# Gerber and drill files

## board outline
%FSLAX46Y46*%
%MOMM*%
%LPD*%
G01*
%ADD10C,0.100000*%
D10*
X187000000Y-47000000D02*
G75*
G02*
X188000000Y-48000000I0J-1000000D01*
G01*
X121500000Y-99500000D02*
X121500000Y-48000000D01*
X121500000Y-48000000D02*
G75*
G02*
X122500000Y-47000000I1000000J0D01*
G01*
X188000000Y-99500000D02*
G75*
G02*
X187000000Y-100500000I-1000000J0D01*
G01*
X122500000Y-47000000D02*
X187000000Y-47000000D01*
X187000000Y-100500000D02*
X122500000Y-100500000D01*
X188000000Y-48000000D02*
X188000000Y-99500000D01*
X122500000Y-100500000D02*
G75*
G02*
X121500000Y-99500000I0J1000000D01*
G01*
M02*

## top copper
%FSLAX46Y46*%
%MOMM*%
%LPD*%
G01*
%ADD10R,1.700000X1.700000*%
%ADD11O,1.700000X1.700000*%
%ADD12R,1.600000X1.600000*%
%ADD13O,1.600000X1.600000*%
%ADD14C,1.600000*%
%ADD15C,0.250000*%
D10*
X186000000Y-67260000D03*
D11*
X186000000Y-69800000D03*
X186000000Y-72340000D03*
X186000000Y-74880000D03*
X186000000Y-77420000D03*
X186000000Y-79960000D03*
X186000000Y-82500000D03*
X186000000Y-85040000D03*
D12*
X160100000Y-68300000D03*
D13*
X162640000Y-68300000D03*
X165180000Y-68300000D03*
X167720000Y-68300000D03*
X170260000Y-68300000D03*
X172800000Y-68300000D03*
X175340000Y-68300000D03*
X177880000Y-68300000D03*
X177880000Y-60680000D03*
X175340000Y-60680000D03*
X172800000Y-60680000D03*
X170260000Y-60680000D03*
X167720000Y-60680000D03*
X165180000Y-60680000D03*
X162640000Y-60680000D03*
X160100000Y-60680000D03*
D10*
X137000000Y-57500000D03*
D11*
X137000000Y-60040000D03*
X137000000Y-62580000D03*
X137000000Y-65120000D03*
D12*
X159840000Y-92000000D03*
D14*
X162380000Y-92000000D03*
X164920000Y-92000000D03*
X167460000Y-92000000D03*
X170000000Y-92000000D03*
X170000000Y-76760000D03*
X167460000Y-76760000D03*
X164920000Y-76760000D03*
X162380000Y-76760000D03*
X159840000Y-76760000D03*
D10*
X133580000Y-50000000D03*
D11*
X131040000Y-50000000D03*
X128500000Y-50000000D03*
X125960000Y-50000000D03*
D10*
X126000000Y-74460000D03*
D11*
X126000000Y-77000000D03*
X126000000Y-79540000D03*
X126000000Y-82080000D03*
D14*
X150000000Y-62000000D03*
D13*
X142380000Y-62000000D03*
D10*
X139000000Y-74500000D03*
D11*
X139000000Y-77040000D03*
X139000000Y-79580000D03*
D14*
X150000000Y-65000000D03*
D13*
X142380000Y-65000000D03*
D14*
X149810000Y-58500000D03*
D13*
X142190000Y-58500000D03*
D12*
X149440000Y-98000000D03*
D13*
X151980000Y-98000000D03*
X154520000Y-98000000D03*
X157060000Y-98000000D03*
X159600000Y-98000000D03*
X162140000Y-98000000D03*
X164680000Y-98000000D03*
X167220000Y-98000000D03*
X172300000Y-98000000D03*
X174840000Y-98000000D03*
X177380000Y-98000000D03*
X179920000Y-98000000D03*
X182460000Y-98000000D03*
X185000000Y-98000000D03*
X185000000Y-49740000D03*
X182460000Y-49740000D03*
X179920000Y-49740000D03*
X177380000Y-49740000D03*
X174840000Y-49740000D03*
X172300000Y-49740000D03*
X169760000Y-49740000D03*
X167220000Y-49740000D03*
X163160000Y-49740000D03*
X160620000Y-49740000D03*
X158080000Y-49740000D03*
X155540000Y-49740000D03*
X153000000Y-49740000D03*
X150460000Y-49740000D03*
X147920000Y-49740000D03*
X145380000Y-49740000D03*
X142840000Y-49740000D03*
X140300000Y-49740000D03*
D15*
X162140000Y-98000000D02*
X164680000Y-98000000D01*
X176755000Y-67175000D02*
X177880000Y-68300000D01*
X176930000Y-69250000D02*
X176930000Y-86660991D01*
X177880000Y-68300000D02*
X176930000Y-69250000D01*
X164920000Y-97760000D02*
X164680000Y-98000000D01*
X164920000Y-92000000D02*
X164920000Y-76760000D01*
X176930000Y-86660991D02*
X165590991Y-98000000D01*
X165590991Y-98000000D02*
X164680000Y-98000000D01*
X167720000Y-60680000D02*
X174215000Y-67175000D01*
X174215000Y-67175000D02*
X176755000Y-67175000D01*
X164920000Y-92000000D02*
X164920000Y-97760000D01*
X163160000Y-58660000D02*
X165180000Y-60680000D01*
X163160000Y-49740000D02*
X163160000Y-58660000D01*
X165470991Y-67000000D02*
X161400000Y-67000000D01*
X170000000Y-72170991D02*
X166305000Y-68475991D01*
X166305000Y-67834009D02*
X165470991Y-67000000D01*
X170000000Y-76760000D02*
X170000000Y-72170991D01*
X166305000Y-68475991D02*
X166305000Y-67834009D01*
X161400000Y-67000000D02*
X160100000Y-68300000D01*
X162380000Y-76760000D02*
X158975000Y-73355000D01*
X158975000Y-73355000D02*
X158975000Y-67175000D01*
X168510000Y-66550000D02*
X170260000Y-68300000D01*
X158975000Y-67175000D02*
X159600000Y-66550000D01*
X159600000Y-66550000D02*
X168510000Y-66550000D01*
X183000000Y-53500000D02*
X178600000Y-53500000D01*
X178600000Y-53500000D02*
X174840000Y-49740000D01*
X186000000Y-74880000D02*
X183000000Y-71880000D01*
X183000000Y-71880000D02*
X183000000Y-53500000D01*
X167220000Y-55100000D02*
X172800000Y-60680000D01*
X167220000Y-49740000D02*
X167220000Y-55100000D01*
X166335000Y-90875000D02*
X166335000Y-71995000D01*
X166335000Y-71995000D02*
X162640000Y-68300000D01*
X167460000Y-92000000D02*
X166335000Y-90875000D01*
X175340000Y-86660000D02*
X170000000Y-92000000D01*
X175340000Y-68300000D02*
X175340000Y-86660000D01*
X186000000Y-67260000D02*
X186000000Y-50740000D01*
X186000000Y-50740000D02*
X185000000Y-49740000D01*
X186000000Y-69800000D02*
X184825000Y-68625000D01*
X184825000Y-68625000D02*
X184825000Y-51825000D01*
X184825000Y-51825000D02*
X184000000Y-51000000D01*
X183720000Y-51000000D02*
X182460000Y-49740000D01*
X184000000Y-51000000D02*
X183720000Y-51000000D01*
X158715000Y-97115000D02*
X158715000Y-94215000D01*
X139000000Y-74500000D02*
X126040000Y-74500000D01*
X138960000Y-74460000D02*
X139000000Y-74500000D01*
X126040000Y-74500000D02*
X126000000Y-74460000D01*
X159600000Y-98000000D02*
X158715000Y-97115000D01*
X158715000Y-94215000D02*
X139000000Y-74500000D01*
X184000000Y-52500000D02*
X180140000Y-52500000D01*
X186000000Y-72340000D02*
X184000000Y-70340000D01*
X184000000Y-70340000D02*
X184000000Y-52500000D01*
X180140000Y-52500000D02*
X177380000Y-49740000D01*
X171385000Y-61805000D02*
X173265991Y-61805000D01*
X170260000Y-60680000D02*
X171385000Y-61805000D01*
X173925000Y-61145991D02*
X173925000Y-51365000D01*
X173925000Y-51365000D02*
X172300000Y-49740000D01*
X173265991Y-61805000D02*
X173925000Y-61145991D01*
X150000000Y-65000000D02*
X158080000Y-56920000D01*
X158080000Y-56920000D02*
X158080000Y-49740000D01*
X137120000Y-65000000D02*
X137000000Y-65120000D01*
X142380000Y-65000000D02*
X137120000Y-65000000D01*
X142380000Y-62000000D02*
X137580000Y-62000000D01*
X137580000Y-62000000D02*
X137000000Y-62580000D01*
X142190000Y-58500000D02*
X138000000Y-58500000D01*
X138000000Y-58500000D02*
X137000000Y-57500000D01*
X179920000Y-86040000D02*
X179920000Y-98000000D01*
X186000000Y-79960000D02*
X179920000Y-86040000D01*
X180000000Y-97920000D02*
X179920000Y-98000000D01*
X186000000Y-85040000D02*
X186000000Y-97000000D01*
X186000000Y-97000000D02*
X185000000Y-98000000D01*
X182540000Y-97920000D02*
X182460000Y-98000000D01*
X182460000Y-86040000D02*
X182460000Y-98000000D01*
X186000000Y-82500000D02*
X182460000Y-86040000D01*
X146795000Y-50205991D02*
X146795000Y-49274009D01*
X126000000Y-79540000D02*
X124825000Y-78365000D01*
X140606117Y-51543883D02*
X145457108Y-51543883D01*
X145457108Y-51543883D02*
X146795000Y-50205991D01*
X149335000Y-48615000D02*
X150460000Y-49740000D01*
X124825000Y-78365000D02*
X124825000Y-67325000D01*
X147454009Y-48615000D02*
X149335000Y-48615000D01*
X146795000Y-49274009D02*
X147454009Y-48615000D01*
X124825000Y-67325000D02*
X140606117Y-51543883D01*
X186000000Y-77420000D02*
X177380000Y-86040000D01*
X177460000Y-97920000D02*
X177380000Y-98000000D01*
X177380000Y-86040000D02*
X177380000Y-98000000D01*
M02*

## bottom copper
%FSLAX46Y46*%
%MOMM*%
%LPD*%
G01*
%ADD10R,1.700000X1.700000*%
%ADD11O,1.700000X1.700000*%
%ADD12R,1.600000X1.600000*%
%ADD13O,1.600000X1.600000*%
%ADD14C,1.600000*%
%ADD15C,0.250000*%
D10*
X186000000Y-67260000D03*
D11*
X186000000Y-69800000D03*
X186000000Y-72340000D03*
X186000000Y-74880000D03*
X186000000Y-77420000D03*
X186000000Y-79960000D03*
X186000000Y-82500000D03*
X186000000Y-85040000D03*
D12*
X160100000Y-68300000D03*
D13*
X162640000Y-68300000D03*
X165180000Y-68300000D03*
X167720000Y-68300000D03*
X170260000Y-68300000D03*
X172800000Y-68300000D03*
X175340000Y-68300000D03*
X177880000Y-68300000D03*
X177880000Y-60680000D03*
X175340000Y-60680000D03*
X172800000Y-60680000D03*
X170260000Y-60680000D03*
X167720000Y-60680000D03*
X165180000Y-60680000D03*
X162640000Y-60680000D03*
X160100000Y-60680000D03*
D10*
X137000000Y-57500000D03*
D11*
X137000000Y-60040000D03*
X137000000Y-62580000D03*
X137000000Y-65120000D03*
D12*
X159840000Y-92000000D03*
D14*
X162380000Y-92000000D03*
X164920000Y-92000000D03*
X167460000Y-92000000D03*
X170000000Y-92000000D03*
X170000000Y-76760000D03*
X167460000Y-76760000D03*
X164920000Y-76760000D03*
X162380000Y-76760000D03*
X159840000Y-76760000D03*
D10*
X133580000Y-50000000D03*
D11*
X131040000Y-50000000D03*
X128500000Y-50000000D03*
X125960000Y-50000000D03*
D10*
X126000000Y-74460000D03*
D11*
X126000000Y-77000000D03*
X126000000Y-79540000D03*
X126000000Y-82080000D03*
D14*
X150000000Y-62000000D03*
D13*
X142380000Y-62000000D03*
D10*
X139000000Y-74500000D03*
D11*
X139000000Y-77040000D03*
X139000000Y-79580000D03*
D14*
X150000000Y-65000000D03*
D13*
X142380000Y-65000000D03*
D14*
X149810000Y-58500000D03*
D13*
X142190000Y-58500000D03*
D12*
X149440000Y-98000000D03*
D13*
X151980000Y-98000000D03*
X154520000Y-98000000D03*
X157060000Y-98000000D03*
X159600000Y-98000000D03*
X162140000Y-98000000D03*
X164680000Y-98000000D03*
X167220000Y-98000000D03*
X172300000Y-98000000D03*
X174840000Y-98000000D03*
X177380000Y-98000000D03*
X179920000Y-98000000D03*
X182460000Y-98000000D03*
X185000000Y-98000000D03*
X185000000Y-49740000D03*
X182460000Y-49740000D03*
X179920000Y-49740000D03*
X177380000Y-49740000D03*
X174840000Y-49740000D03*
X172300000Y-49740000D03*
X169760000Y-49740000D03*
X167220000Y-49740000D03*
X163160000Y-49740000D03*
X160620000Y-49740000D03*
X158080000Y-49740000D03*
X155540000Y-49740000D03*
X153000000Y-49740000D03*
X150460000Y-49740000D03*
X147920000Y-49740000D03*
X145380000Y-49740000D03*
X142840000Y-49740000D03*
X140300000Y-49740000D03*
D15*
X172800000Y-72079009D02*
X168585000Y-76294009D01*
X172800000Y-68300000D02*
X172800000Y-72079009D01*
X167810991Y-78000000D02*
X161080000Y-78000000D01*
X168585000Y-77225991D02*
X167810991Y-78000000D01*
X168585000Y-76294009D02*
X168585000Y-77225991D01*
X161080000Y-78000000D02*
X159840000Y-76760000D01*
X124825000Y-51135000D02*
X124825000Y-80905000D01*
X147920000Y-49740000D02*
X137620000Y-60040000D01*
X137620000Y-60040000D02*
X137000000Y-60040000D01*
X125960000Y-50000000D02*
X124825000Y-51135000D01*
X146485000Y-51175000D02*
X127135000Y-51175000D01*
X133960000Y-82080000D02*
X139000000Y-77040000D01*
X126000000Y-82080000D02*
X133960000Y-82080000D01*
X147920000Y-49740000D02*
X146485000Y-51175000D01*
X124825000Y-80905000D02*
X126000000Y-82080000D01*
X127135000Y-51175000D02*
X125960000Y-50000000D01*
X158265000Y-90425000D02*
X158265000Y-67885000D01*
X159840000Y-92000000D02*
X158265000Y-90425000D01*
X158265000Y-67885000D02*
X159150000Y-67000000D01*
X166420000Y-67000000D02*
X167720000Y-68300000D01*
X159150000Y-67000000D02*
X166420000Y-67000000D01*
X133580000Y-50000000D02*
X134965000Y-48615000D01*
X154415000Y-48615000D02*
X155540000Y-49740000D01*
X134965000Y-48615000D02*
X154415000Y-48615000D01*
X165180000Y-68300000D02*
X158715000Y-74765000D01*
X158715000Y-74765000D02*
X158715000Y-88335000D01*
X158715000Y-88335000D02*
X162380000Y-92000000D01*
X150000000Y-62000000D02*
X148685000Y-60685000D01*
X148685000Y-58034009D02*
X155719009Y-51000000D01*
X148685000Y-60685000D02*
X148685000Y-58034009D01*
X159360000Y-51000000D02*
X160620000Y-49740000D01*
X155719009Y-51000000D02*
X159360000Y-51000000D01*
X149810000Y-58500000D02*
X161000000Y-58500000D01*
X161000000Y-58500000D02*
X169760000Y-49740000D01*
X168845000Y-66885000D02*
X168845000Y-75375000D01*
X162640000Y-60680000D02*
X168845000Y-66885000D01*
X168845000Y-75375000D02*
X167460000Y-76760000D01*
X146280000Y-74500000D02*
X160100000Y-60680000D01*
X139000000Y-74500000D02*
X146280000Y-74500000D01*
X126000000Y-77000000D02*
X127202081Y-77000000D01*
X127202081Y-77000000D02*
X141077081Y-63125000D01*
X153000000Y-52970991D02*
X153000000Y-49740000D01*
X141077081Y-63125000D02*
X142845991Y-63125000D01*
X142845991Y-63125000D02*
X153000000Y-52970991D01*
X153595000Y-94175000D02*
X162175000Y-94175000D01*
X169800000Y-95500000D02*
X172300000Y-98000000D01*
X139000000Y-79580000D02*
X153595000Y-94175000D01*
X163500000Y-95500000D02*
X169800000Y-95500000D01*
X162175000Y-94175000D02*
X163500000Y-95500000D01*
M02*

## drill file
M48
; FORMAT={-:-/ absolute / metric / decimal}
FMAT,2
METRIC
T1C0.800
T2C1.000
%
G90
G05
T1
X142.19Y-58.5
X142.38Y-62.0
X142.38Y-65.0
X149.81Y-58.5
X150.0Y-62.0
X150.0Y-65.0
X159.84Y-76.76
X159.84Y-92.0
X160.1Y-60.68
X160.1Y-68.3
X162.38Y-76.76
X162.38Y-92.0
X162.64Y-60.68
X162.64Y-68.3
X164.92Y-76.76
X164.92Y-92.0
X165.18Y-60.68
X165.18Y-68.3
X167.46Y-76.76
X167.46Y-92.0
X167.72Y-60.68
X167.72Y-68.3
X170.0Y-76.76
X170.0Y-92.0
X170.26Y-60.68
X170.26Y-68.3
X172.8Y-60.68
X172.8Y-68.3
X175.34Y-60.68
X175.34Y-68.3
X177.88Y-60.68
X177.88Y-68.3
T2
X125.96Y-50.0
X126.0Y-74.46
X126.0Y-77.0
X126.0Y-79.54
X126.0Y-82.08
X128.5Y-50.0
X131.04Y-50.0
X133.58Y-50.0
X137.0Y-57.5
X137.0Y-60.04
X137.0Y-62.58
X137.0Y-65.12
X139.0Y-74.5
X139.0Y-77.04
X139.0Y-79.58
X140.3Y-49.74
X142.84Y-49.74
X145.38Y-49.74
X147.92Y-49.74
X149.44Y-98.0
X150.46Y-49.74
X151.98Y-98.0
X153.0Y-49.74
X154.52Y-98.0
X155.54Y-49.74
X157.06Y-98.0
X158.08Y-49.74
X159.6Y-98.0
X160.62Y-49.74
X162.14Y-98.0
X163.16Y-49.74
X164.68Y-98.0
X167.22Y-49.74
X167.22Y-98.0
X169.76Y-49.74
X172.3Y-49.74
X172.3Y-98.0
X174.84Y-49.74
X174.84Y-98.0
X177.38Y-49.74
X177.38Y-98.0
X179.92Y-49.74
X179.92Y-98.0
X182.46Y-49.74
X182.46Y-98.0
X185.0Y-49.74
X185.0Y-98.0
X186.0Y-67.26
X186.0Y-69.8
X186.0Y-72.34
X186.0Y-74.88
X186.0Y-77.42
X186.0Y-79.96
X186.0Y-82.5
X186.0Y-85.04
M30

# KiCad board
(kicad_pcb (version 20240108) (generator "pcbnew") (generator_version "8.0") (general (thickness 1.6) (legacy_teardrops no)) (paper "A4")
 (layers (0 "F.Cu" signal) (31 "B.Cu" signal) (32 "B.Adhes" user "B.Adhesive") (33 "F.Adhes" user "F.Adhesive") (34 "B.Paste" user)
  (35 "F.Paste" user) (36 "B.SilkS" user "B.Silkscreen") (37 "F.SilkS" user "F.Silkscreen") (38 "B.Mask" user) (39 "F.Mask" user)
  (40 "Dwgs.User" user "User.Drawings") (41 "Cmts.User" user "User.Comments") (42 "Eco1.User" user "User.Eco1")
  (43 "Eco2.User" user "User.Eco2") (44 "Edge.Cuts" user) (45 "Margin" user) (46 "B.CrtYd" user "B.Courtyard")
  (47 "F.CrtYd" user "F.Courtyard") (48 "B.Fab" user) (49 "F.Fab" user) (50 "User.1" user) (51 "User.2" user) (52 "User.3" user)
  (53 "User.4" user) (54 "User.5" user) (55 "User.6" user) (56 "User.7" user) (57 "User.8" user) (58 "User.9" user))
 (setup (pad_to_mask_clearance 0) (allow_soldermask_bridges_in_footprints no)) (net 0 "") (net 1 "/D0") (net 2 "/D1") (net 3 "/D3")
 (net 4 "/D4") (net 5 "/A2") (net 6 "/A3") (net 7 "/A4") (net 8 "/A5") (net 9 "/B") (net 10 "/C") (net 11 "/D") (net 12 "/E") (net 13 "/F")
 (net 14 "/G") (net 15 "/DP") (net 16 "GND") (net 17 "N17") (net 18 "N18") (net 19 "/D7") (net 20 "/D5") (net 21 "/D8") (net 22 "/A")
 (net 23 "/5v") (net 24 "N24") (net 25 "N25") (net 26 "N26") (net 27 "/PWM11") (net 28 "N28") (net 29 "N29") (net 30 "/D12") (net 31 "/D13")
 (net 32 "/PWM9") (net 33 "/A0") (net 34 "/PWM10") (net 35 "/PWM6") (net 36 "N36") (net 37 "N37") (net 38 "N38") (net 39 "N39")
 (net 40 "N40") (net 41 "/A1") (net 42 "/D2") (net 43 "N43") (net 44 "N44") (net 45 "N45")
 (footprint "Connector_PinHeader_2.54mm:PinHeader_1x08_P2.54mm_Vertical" (layer "F.Cu") (at 186 67.26)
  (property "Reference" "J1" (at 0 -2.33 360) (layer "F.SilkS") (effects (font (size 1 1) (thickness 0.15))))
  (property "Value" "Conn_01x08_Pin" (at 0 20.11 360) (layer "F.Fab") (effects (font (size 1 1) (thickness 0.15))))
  (pad "1" thru_hole rect (at 0 0) (size 1.7 1.7) (drill 1) (layers "*.Cu" "*.Mask") (remove_unused_layers no) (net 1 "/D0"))
  (pad "2" thru_hole oval (at 0 2.54) (size 1.7 1.7) (drill 1) (layers "*.Cu" "*.Mask") (remove_unused_layers no) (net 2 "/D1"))
  (pad "3" thru_hole oval (at 0 5.08) (size 1.7 1.7) (drill 1) (layers "*.Cu" "*.Mask") (remove_unused_layers no) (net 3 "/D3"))
  (pad "4" thru_hole oval (at 0 7.62) (size 1.7 1.7) (drill 1) (layers "*.Cu" "*.Mask") (remove_unused_layers no) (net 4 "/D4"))
  (pad "5" thru_hole oval (at 0 10.16) (size 1.7 1.7) (drill 1) (layers "*.Cu" "*.Mask") (remove_unused_layers no) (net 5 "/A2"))
  (pad "6" thru_hole oval (at 0 12.7) (size 1.7 1.7) (drill 1) (layers "*.Cu" "*.Mask") (remove_unused_layers no) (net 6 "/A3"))
  (pad "7" thru_hole oval (at 0 15.24) (size 1.7 1.7) (drill 1) (layers "*.Cu" "*.Mask") (remove_unused_layers no) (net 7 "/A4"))
  (pad "8" thru_hole oval (at 0 17.78) (size 1.7 1.7) (drill 1) (layers "*.Cu" "*.Mask") (remove_unused_layers no) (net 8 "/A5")))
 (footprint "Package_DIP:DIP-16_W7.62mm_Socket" (layer "F.Cu") (at 160.1 68.3 90)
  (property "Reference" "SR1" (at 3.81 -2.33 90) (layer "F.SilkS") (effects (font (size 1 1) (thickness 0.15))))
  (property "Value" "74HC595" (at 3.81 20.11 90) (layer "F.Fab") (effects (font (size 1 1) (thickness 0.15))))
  (pad "1" thru_hole rect (at 0 0 90) (size 1.6 1.6) (drill 0.8) (layers "*.Cu" "*.Mask") (remove_unused_layers no) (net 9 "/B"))
  (pad "2" thru_hole oval (at 0 2.54 90) (size 1.6 1.6) (drill 0.8) (layers "*.Cu" "*.Mask") (remove_unused_layers no) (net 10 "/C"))
  (pad "3" thru_hole oval (at 0 5.08 90) (size 1.6 1.6) (drill 0.8) (layers "*.Cu" "*.Mask") (remove_unused_layers no) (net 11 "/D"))
  (pad "4" thru_hole oval (at 0 7.62 90) (size 1.6 1.6) (drill 0.8) (layers "*.Cu" "*.Mask") (remove_unused_layers no) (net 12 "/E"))
  (pad "5" thru_hole oval (at 0 10.16 90) (size 1.6 1.6) (drill 0.8) (layers "*.Cu" "*.Mask") (remove_unused_layers no) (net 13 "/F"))
  (pad "6" thru_hole oval (at 0 12.7 90) (size 1.6 1.6) (drill 0.8) (layers "*.Cu" "*.Mask") (remove_unused_layers no) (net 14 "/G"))
  (pad "7" thru_hole oval (at 0 15.24 90) (size 1.6 1.6) (drill 0.8) (layers "*.Cu" "*.Mask") (remove_unused_layers no) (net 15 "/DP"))
  (pad "8" thru_hole oval (at 0 17.78 90) (size 1.6 1.6) (drill 0.8) (layers "*.Cu" "*.Mask") (remove_unused_layers no) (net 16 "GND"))
  (pad "9" thru_hole oval (at 7.62 17.78 90) (size 1.6 1.6) (drill 0.8) (layers "*.Cu" "*.Mask") (remove_unused_layers no) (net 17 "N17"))
  (pad "10" thru_hole oval (at 7.62 15.24 90) (size 1.6 1.6) (drill 0.8) (layers "*.Cu" "*.Mask") (remove_unused_layers no) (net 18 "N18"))
  (pad "11" thru_hole oval (at 7.62 12.7 90) (size 1.6 1.6) (drill 0.8) (layers "*.Cu" "*.Mask") (remove_unused_layers no) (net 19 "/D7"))
  (pad "12" thru_hole oval (at 7.62 10.16 90) (size 1.6 1.6) (drill 0.8) (layers "*.Cu" "*.Mask") (remove_unused_layers no) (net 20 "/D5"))
  (pad "13" thru_hole oval (at 7.62 7.62 90) (size 1.6 1.6) (drill 0.8) (layers "*.Cu" "*.Mask") (remove_unused_layers no) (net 16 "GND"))
  (pad "14" thru_hole oval (at 7.62 5.08 90) (size 1.6 1.6) (drill 0.8) (layers "*.Cu" "*.Mask") (remove_unused_layers no) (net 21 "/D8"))
  (pad "15" thru_hole oval (at 7.62 2.54 90) (size 1.6 1.6) (drill 0.8) (layers "*.Cu" "*.Mask") (remove_unused_layers no) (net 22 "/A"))
  (pad "16" thru_hole oval (at 7.62 0 90) (size 1.6 1.6) (drill 0.8) (layers "*.Cu" "*.Mask") (remove_unused_layers no) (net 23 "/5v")))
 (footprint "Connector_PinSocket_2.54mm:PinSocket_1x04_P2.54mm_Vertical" (layer "F.Cu") (at 137 57.5)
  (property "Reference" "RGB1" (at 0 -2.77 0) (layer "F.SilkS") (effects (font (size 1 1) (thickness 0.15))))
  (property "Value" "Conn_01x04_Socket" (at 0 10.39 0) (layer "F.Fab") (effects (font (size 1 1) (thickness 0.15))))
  (pad "1" thru_hole rect (at 0 0) (size 1.7 1.7) (drill 1) (layers "*.Cu" "*.Mask") (remove_unused_layers no) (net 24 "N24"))
  (pad "2" thru_hole oval (at 0 2.54) (size 1.7 1.7) (drill 1) (layers "*.Cu" "*.Mask") (remove_unused_layers no) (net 16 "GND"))
  (pad "3" thru_hole oval (at 0 5.08) (size 1.7 1.7) (drill 1) (layers "*.Cu" "*.Mask") (remove_unused_layers no) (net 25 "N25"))
  (pad "4" thru_hole oval (at 0 7.62) (size 1.7 1.7) (drill 1) (layers "*.Cu" "*.Mask") (remove_unused_layers no) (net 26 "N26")))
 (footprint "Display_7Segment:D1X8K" (layer "F.Cu") (at 159.84 92 90)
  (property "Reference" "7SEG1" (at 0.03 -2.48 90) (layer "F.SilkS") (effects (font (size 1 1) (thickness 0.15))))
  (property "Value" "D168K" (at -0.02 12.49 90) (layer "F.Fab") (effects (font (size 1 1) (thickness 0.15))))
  (pad "1" thru_hole rect (at 0 0) (size 1.6 1.6) (drill 0.8) (layers "*.Cu" "*.Mask") (remove_unused_layers no) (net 12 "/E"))
  (pad "2" thru_hole circle (at 0 2.54) (size 1.6 1.6) (drill 0.8) (layers "*.Cu" "*.Mask") (remove_unused_layers no) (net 11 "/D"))
  (pad "3" thru_hole circle (at 0 5.08) (size 1.6 1.6) (drill 0.8) (layers "*.Cu" "*.Mask") (remove_unused_layers no) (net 16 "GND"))
  (pad "4" thru_hole circle (at 0 7.62) (size 1.6 1.6) (drill 0.8) (layers "*.Cu" "*.Mask") (remove_unused_layers no) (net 10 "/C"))
  (pad "5" thru_hole circle (at 0 10.16) (size 1.6 1.6) (drill 0.8) (layers "*.Cu" "*.Mask") (remove_unused_layers no) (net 15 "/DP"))
  (pad "6" thru_hole circle (at 15.24 10.16) (size 1.6 1.6) (drill 0.8) (layers "*.Cu" "*.Mask") (remove_unused_layers no) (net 9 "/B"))
  (pad "7" thru_hole circle (at 15.24 7.62) (size 1.6 1.6) (drill 0.8) (layers "*.Cu" "*.Mask") (remove_unused_layers no) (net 22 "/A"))
  (pad "8" thru_hole circle (at 15.24 5.08) (size 1.6 1.6) (drill 0.8) (layers "*.Cu" "*.Mask") (remove_unused_layers no) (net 16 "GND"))
  (pad "9" thru_hole circle (at 15.24 2.54) (size 1.6 1.6) (drill 0.8) (layers "*.Cu" "*.Mask") (remove_unused_layers no) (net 13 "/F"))
  (pad "10" thru_hole circle (at 15.24 0) (size 1.6 1.6) (drill 0.8) (layers "*.Cu" "*.Mask") (remove_unused_layers no) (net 14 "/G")))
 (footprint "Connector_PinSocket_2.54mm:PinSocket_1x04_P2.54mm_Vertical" (layer "F.Cu") (at 133.58 50 -90)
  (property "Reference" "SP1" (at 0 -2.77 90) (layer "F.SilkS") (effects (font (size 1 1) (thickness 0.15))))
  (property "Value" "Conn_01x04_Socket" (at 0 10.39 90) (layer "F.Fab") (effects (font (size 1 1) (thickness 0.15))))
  (pad "1" thru_hole rect (at 0 0 270) (size 1.7 1.7) (drill 1) (layers "*.Cu" "*.Mask") (remove_unused_layers no) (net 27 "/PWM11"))
  (pad "2" thru_hole oval (at 0 2.54 270) (size 1.7 1.7) (drill 1) (layers "*.Cu" "*.Mask") (remove_unused_layers no) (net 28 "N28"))
  (pad "3" thru_hole oval (at 0 5.08 270) (size 1.7 1.7) (drill 1) (layers "*.Cu" "*.Mask") (remove_unused_layers no) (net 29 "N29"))
  (pad "4" thru_hole oval (at 0 7.62 270) (size 1.7 1.7) (drill 1) (layers "*.Cu" "*.Mask") (remove_unused_layers no) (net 16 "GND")))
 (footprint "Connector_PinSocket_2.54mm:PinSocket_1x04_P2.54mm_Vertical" (layer "F.Cu") (at 126 74.46)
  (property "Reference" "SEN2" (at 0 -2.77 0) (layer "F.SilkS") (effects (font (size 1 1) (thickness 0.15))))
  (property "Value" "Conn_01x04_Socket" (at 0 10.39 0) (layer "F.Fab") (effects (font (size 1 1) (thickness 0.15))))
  (pad "1" thru_hole rect (at 0 0) (size 1.7 1.7) (drill 1) (layers "*.Cu" "*.Mask") (remove_unused_layers no) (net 23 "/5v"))
  (pad "2" thru_hole oval (at 0 2.54) (size 1.7 1.7) (drill 1) (layers "*.Cu" "*.Mask") (remove_unused_layers no) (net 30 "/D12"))
  (pad "3" thru_hole oval (at 0 5.08) (size 1.7 1.7) (drill 1) (layers "*.Cu" "*.Mask") (remove_unused_layers no) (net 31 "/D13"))
  (pad "4" thru_hole oval (at 0 7.62) (size 1.7 1.7) (drill 1) (layers "*.Cu" "*.Mask") (remove_unused_layers no) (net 16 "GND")))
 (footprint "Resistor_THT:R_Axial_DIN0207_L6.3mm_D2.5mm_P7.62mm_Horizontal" (layer "F.Cu") (at 150 62 180)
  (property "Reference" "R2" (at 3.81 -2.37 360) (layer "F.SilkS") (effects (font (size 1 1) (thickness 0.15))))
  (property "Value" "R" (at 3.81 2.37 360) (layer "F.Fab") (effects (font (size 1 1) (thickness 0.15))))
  (pad "1" thru_hole circle (at 0 0 180) (size 1.6 1.6) (drill 0.8) (layers "*.Cu" "*.Mask") (remove_unused_layers no) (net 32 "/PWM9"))
  (pad "2" thru_hole oval (at 7.62 0 180) (size 1.6 1.6) (drill 0.8) (layers "*.Cu" "*.Mask") (remove_unused_layers no) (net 25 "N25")))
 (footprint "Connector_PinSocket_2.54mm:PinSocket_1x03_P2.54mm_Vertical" (layer "F.Cu") (at 139 74.5)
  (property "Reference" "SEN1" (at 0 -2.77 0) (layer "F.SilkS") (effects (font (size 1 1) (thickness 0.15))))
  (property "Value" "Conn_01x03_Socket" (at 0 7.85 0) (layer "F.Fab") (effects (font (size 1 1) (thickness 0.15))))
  (pad "1" thru_hole rect (at 0 0) (size 1.7 1.7) (drill 1) (layers "*.Cu" "*.Mask") (remove_unused_layers no) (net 23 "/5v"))
  (pad "2" thru_hole oval (at 0 2.54) (size 1.7 1.7) (drill 1) (layers "*.Cu" "*.Mask") (remove_unused_layers no) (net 16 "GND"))
  (pad "3" thru_hole oval (at 0 5.08) (size 1.7 1.7) (drill 1) (layers "*.Cu" "*.Mask") (remove_unused_layers no) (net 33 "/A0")))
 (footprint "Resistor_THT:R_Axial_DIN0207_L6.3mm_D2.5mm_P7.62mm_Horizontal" (layer "F.Cu") (at 150 65 180)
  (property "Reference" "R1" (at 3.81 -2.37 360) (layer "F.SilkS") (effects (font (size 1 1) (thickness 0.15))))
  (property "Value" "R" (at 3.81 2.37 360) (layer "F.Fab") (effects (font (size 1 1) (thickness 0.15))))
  (pad "1" thru_hole circle (at 0 0 180) (size 1.6 1.6) (drill 0.8) (layers "*.Cu" "*.Mask") (remove_unused_layers no) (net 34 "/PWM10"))
  (pad "2" thru_hole oval (at 7.62 0 180) (size 1.6 1.6) (drill 0.8) (layers "*.Cu" "*.Mask") (remove_unused_layers no) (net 26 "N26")))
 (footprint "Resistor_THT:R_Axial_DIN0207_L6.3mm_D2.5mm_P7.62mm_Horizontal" (layer "F.Cu") (at 149.81 58.5 180)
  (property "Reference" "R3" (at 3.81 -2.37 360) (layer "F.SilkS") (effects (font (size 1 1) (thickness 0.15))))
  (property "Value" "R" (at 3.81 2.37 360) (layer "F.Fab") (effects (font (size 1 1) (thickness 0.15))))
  (pad "1" thru_hole circle (at 0 0 180) (size 1.6 1.6) (drill 0.8) (layers "*.Cu" "*.Mask") (remove_unused_layers no) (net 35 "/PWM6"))
  (pad "2" thru_hole oval (at 7.62 0 180) (size 1.6 1.6) (drill 0.8) (layers "*.Cu" "*.Mask") (remove_unused_layers no) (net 24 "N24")))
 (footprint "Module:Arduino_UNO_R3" (layer "B.Cu") (at 149.44 98)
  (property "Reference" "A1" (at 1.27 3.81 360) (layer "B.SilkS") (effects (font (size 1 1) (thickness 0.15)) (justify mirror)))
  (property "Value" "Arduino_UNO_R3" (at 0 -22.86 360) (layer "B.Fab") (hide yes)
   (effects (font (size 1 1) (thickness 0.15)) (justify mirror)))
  (pad "1" thru_hole rect (at 0 0 270) (size 1.6 1.6) (drill 1) (layers "*.Cu" "*.Mask") (remove_unused_layers no) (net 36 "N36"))
  (pad "2" thru_hole oval (at 2.54 0 270) (size 1.6 1.6) (drill 1) (layers "*.Cu" "*.Mask") (remove_unused_layers no) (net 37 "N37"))
  (pad "3" thru_hole oval (at 5.08 0 270) (size 1.6 1.6) (drill 1) (layers "*.Cu" "*.Mask") (remove_unused_layers no) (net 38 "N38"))
  (pad "4" thru_hole oval (at 7.62 0 270) (size 1.6 1.6) (drill 1) (layers "*.Cu" "*.Mask") (remove_unused_layers no) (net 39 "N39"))
  (pad "5" thru_hole oval (at 10.16 0 270) (size 1.6 1.6) (drill 1) (layers "*.Cu" "*.Mask") (remove_unused_layers no) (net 23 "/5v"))
  (pad "6" thru_hole oval (at 12.7 0 270) (size 1.6 1.6) (drill 1) (layers "*.Cu" "*.Mask") (remove_unused_layers no) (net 16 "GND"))
  (pad "7" thru_hole oval (at 15.24 0 270) (size 1.6 1.6) (drill 1) (layers "*.Cu" "*.Mask") (remove_unused_layers no) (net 16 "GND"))
  (pad "8" thru_hole oval (at 17.78 0 270) (size 1.6 1.6) (drill 1) (layers "*.Cu" "*.Mask") (remove_unused_layers no) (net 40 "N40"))
  (pad "9" thru_hole oval (at 22.86 0 270) (size 1.6 1.6) (drill 1) (layers "*.Cu" "*.Mask") (remove_unused_layers no) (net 33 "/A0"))
  (pad "10" thru_hole oval (at 25.4 0 270) (size 1.6 1.6) (drill 1) (layers "*.Cu" "*.Mask") (remove_unused_layers no) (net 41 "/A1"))
  (pad "11" thru_hole oval (at 27.94 0 270) (size 1.6 1.6) (drill 1) (layers "*.Cu" "*.Mask") (remove_unused_layers no) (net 5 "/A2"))
  (pad "12" thru_hole oval (at 30.48 0 270) (size 1.6 1.6) (drill 1) (layers "*.Cu" "*.Mask") (remove_unused_layers no) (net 6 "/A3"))
  (pad "13" thru_hole oval (at 33.02 0 270) (size 1.6 1.6) (drill 1) (layers "*.Cu" "*.Mask") (remove_unused_layers no) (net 7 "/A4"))
  (pad "14" thru_hole oval (at 35.56 0 270) (size 1.6 1.6) (drill 1) (layers "*.Cu" "*.Mask") (remove_unused_layers no) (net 8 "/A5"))
  (pad "15" thru_hole oval (at 35.56 -48.26 270) (size 1.6 1.6) (drill 1) (layers "*.Cu" "*.Mask") (remove_unused_layers no) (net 1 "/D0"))
  (pad "16" thru_hole oval (at 33.02 -48.26 270) (size 1.6 1.6) (drill 1) (layers "*.Cu" "*.Mask") (remove_unused_layers no) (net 2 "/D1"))
  (pad "17" thru_hole oval (at 30.48 -48.26 270) (size 1.6 1.6) (drill 1) (layers "*.Cu" "*.Mask") (remove_unused_layers no) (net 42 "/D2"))
  (pad "18" thru_hole oval (at 27.94 -48.26 270) (size 1.6 1.6) (drill 1) (layers "*.Cu" "*.Mask") (remove_unused_layers no) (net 3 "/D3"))
  (pad "19" thru_hole oval (at 25.4 -48.26 270) (size 1.6 1.6) (drill 1) (layers "*.Cu" "*.Mask") (remove_unused_layers no) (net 4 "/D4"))
  (pad "20" thru_hole oval (at 22.86 -48.26 270) (size 1.6 1.6) (drill 1) (layers "*.Cu" "*.Mask") (remove_unused_layers no) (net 20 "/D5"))
  (pad "21" thru_hole oval (at 20.32 -48.26 270) (size 1.6 1.6) (drill 1) (layers "*.Cu" "*.Mask") (remove_unused_layers no)
   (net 35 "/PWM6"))
  (pad "22" thru_hole oval (at 17.78 -48.26 270) (size 1.6 1.6) (drill 1) (layers "*.Cu" "*.Mask") (remove_unused_layers no) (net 19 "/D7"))
  (pad "23" thru_hole oval (at 13.72 -48.26 270) (size 1.6 1.6) (drill 1) (layers "*.Cu" "*.Mask") (remove_unused_layers no) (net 21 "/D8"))
  (pad "24" thru_hole oval (at 11.18 -48.26 270) (size 1.6 1.6) (drill 1) (layers "*.Cu" "*.Mask") (remove_unused_layers no)
   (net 32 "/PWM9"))
  (pad "25" thru_hole oval (at 8.64 -48.26 270) (size 1.6 1.6) (drill 1) (layers "*.Cu" "*.Mask") (remove_unused_layers no)
   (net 34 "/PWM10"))
  (pad "26" thru_hole oval (at 6.1 -48.26 270) (size 1.6 1.6) (drill 1) (layers "*.Cu" "*.Mask") (remove_unused_layers no) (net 27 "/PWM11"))
  (pad "27" thru_hole oval (at 3.56 -48.26 270) (size 1.6 1.6) (drill 1) (layers "*.Cu" "*.Mask") (remove_unused_layers no) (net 30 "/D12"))
  (pad "28" thru_hole oval (at 1.02 -48.26 270) (size 1.6 1.6) (drill 1) (layers "*.Cu" "*.Mask") (remove_unused_layers no) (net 31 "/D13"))
  (pad "29" thru_hole oval (at -1.52 -48.26 270) (size 1.6 1.6) (drill 1) (layers "*.Cu" "*.Mask") (remove_unused_layers no) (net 16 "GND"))
  (pad "30" thru_hole oval (at -4.06 -48.26 270) (size 1.6 1.6) (drill 1) (layers "*.Cu" "*.Mask") (remove_unused_layers no) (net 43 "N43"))
  (pad "31" thru_hole oval (at -6.6 -48.26 270) (size 1.6 1.6) (drill 1) (layers "*.Cu" "*.Mask") (remove_unused_layers no) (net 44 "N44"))
  (pad "32" thru_hole oval (at -9.14 -48.26 270) (size 1.6 1.6) (drill 1) (layers "*.Cu" "*.Mask") (remove_unused_layers no) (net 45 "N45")))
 (gr_arc (start 187 47) (mid 187.707107 47.292893) (end 188 48) (stroke (width 0.1) (type default)) (layer "Edge.Cuts"))
 (gr_line (start 121.5 99.5) (end 121.5 48) (stroke (width 0.1) (type default)) (layer "Edge.Cuts"))
 (gr_arc (start 121.5 48) (mid 121.792893 47.292893) (end 122.5 47) (stroke (width 0.1) (type default)) (layer "Edge.Cuts"))
 (gr_arc (start 188 99.5) (mid 187.707107 100.207107) (end 187 100.5) (stroke (width 0.1) (type default)) (layer "Edge.Cuts"))
 (gr_line (start 122.5 47) (end 187 47) (stroke (width 0.1) (type default)) (layer "Edge.Cuts"))
 (gr_line (start 187 100.5) (end 122.5 100.5) (stroke (width 0.1) (type default)) (layer "Edge.Cuts"))
 (gr_line (start 188 48) (end 188 99.5) (stroke (width 0.1) (type default)) (layer "Edge.Cuts"))
 (gr_arc (start 122.5 100.5) (mid 121.792893 100.207107) (end 121.5 99.5) (stroke (width 0.1) (type default)) (layer "Edge.Cuts"))
 (segment (start 172.8 72.079009) (end 168.585 76.294009) (width 0.25) (layer "B.Cu") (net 14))
 (segment (start 172.8 68.3) (end 172.8 72.079009) (width 0.25) (layer "B.Cu") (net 14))
 (segment (start 167.810991 78) (end 161.08 78) (width 0.25) (layer "B.Cu") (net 14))
 (segment (start 168.585 77.225991) (end 167.810991 78) (width 0.25) (layer "B.Cu") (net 14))
 (segment (start 168.585 76.294009) (end 168.585 77.225991) (width 0.25) (layer "B.Cu") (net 14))
 (segment (start 161.08 78) (end 159.84 76.76) (width 0.25) (layer "B.Cu") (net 14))
 (segment (start 162.14 98) (end 164.68 98) (width 0.25) (layer "F.Cu") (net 16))
 (segment (start 176.755 67.175) (end 177.88 68.3) (width 0.25) (layer "F.Cu") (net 16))
 (segment (start 176.93 69.25) (end 176.93 86.660991) (width 0.25) (layer "F.Cu") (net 16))
 (segment (start 177.88 68.3) (end 176.93 69.25) (width 0.25) (layer "F.Cu") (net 16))
 (segment (start 164.92 97.76) (end 164.68 98) (width 0.25) (layer "F.Cu") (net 16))
 (segment (start 164.92 92) (end 164.92 76.76) (width 0.25) (layer "F.Cu") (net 16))
 (segment (start 176.93 86.660991) (end 165.590991 98) (width 0.25) (layer "F.Cu") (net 16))
 (segment (start 165.590991 98) (end 164.68 98) (width 0.25) (layer "F.Cu") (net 16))
 (segment (start 167.72 60.68) (end 174.215 67.175) (width 0.25) (layer "F.Cu") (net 16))
 (segment (start 174.215 67.175) (end 176.755 67.175) (width 0.25) (layer "F.Cu") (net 16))
 (segment (start 164.92 92) (end 164.92 97.76) (width 0.25) (layer "F.Cu") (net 16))
 (segment (start 124.825 51.135) (end 124.825 80.905) (width 0.25) (layer "B.Cu") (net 16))
 (segment (start 147.92 49.74) (end 137.62 60.04) (width 0.25) (layer "B.Cu") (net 16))
 (segment (start 137.62 60.04) (end 137 60.04) (width 0.25) (layer "B.Cu") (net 16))
 (segment (start 125.96 50) (end 124.825 51.135) (width 0.25) (layer "B.Cu") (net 16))
 (segment (start 146.485 51.175) (end 127.135 51.175) (width 0.25) (layer "B.Cu") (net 16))
 (segment (start 133.96 82.08) (end 139 77.04) (width 0.25) (layer "B.Cu") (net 16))
 (segment (start 126 82.08) (end 133.96 82.08) (width 0.25) (layer "B.Cu") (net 16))
 (segment (start 147.92 49.74) (end 146.485 51.175) (width 0.25) (layer "B.Cu") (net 16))
 (segment (start 124.825 80.905) (end 126 82.08) (width 0.25) (layer "B.Cu") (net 16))
 (segment (start 127.135 51.175) (end 125.96 50) (width 0.25) (layer "B.Cu") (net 16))
 (segment (start 158.265 90.425) (end 158.265 67.885) (width 0.25) (layer "B.Cu") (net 12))
 (segment (start 159.84 92) (end 158.265 90.425) (width 0.25) (layer "B.Cu") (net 12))
 (segment (start 158.265 67.885) (end 159.15 67) (width 0.25) (layer "B.Cu") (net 12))
 (segment (start 166.42 67) (end 167.72 68.3) (width 0.25) (layer "B.Cu") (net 12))
 (segment (start 159.15 67) (end 166.42 67) (width 0.25) (layer "B.Cu") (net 12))
 (segment (start 163.16 58.66) (end 165.18 60.68) (width 0.25) (layer "F.Cu") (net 21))
 (segment (start 163.16 49.74) (end 163.16 58.66) (width 0.25) (layer "F.Cu") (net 21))
 (segment (start 165.470991 67) (end 161.4 67) (width 0.25) (layer "F.Cu") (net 9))
 (segment (start 170 72.170991) (end 166.305 68.475991) (width 0.25) (layer "F.Cu") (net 9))
 (segment (start 166.305 67.834009) (end 165.470991 67) (width 0.25) (layer "F.Cu") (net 9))
 (segment (start 170 76.76) (end 170 72.170991) (width 0.25) (layer "F.Cu") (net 9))
 (segment (start 166.305 68.475991) (end 166.305 67.834009) (width 0.25) (layer "F.Cu") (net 9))
 (segment (start 161.4 67) (end 160.1 68.3) (width 0.25) (layer "F.Cu") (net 9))
 (segment (start 162.38 76.76) (end 158.975 73.355) (width 0.25) (layer "F.Cu") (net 13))
 (segment (start 158.975 73.355) (end 158.975 67.175) (width 0.25) (layer "F.Cu") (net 13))
 (segment (start 168.51 66.55) (end 170.26 68.3) (width 0.25) (layer "F.Cu") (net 13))
 (segment (start 158.975 67.175) (end 159.6 66.55) (width 0.25) (layer "F.Cu") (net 13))
 (segment (start 159.6 66.55) (end 168.51 66.55) (width 0.25) (layer "F.Cu") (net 13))
 (segment (start 183 53.5) (end 178.6 53.5) (width 0.25) (layer "F.Cu") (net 4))
 (segment (start 178.6 53.5) (end 174.84 49.74) (width 0.25) (layer "F.Cu") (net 4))
 (segment (start 186 74.88) (end 183 71.88) (width 0.25) (layer "F.Cu") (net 4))
 (segment (start 183 71.88) (end 183 53.5) (width 0.25) (layer "F.Cu") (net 4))
 (segment (start 167.22 55.1) (end 172.8 60.68) (width 0.25) (layer "F.Cu") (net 19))
 (segment (start 167.22 49.74) (end 167.22 55.1) (width 0.25) (layer "F.Cu") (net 19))
 (segment (start 133.58 50) (end 134.965 48.615) (width 0.25) (layer "B.Cu") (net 27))
 (segment (start 154.415 48.615) (end 155.54 49.74) (width 0.25) (layer "B.Cu") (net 27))
 (segment (start 134.965 48.615) (end 154.415 48.615) (width 0.25) (layer "B.Cu") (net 27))
 (segment (start 166.335 90.875) (end 166.335 71.995) (width 0.25) (layer "F.Cu") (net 10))
 (segment (start 166.335 71.995) (end 162.64 68.3) (width 0.25) (layer "F.Cu") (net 10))
 (segment (start 167.46 92) (end 166.335 90.875) (width 0.25) (layer "F.Cu") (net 10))
 (segment (start 165.18 68.3) (end 158.715 74.765) (width 0.25) (layer "B.Cu") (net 11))
 (segment (start 158.715 74.765) (end 158.715 88.335) (width 0.25) (layer "B.Cu") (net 11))
 (segment (start 158.715 88.335) (end 162.38 92) (width 0.25) (layer "B.Cu") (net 11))
 (segment (start 150 62) (end 148.685 60.685) (width 0.25) (layer "B.Cu") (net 32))
 (segment (start 148.685 58.034009) (end 155.719009 51) (width 0.25) (layer "B.Cu") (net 32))
 (segment (start 148.685 60.685) (end 148.685 58.034009) (width 0.25) (layer "B.Cu") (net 32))
 (segment (start 159.36 51) (end 160.62 49.74) (width 0.25) (layer "B.Cu") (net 32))
 (segment (start 155.719009 51) (end 159.36 51) (width 0.25) (layer "B.Cu") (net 32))
 (segment (start 149.81 58.5) (end 161 58.5) (width 0.25) (layer "B.Cu") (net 35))
 (segment (start 161 58.5) (end 169.76 49.74) (width 0.25) (layer "B.Cu") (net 35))
 (segment (start 175.34 86.66) (end 170 92) (width 0.25) (layer "F.Cu") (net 15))
 (segment (start 175.34 68.3) (end 175.34 86.66) (width 0.25) (layer "F.Cu") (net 15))
 (segment (start 186 67.26) (end 186 50.74) (width 0.25) (layer "F.Cu") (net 1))
 (segment (start 186 50.74) (end 185 49.74) (width 0.25) (layer "F.Cu") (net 1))
 (segment (start 168.845 66.885) (end 168.845 75.375) (width 0.25) (layer "B.Cu") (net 22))
 (segment (start 162.64 60.68) (end 168.845 66.885) (width 0.25) (layer "B.Cu") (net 22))
 (segment (start 168.845 75.375) (end 167.46 76.76) (width 0.25) (layer "B.Cu") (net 22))
 (segment (start 186 69.8) (end 184.825 68.625) (width 0.25) (layer "F.Cu") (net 2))
 (segment (start 184.825 68.625) (end 184.825 51.825) (width 0.25) (layer "F.Cu") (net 2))
 (segment (start 184.825 51.825) (end 184 51) (width 0.25) (layer "F.Cu") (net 2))
 (segment (start 183.72 51) (end 182.46 49.74) (width 0.25) (layer "F.Cu") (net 2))
 (segment (start 184 51) (end 183.72 51) (width 0.25) (layer "F.Cu") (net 2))
 (segment (start 158.715 97.115) (end 158.715 94.215) (width 0.25) (layer "F.Cu") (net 23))
 (segment (start 139 74.5) (end 126.04 74.5) (width 0.25) (layer "F.Cu") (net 23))
 (segment (start 138.96 74.46) (end 139 74.5) (width 0.25) (layer "F.Cu") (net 23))
 (segment (start 126.04 74.5) (end 126 74.46) (width 0.25) (layer "F.Cu") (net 23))
 (segment (start 159.6 98) (end 158.715 97.115) (width 0.25) (layer "F.Cu") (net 23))
 (segment (start 158.715 94.215) (end 139 74.5) (width 0.25) (layer "F.Cu") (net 23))
 (segment (start 146.28 74.5) (end 160.1 60.68) (width 0.25) (layer "B.Cu") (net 23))
 (segment (start 139 74.5) (end 146.28 74.5) (width 0.25) (layer "B.Cu") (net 23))
 (segment (start 184 52.5) (end 180.14 52.5) (width 0.25) (layer "F.Cu") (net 3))
 (segment (start 186 72.34) (end 184 70.34) (width 0.25) (layer "F.Cu") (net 3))
 (segment (start 184 70.34) (end 184 52.5) (width 0.25) (layer "F.Cu") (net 3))
 (segment (start 180.14 52.5) (end 177.38 49.74) (width 0.25) (layer "F.Cu") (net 3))
 (segment (start 171.385 61.805) (end 173.265991 61.805) (width 0.25) (layer "F.Cu") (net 20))
 (segment (start 170.26 60.68) (end 171.385 61.805) (width 0.25) (layer "F.Cu") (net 20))
 (segment (start 173.925 61.145991) (end 173.925 51.365) (width 0.25) (layer "F.Cu") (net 20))
 (segment (start 173.925 51.365) (end 172.3 49.74) (width 0.25) (layer "F.Cu") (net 20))
 (segment (start 173.265991 61.805) (end 173.925 61.145991) (width 0.25) (layer "F.Cu") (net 20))
 (segment (start 150 65) (end 158.08 56.92) (width 0.25) (layer "F.Cu") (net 34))
 (segment (start 158.08 56.92) (end 158.08 49.74) (width 0.25) (layer "F.Cu") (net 34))
 (segment (start 137.12 65) (end 137 65.12) (width 0.25) (layer "F.Cu") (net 26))
 (segment (start 142.38 65) (end 137.12 65) (width 0.25) (layer "F.Cu") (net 26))
 (segment (start 142.38 62) (end 137.58 62) (width 0.25) (layer "F.Cu") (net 25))
 (segment (start 137.58 62) (end 137 62.58) (width 0.25) (layer "F.Cu") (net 25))
 (segment (start 142.19 58.5) (end 138 58.5) (width 0.25) (layer "F.Cu") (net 24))
 (segment (start 138 58.5) (end 137 57.5) (width 0.25) (layer "F.Cu") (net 24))
 (segment (start 179.92 86.04) (end 179.92 98) (width 0.25) (layer "F.Cu") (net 6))
 (segment (start 186 79.96) (end 179.92 86.04) (width 0.25) (layer "F.Cu") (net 6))
 (segment (start 180 97.92) (end 179.92 98) (width 0.25) (layer "F.Cu") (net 6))
 (segment (start 186 85.04) (end 186 97) (width 0.25) (layer "F.Cu") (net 8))
 (segment (start 186 97) (end 185 98) (width 0.25) (layer "F.Cu") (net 8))
 (segment (start 182.54 97.92) (end 182.46 98) (width 0.25) (layer "F.Cu") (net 7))
 (segment (start 182.46 86.04) (end 182.46 98) (width 0.25) (layer "F.Cu") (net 7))
 (segment (start 186 82.5) (end 182.46 86.04) (width 0.25) (layer "F.Cu") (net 7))
 (segment (start 126 77) (end 127.202081 77) (width 0.25) (layer "B.Cu") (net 30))
 (segment (start 127.202081 77) (end 141.077081 63.125) (width 0.25) (layer "B.Cu") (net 30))
 (segment (start 153 52.970991) (end 153 49.74) (width 0.25) (layer "B.Cu") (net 30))
 (segment (start 141.077081 63.125) (end 142.845991 63.125) (width 0.25) (layer "B.Cu") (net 30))
 (segment (start 142.845991 63.125) (end 153 52.970991) (width 0.25) (layer "B.Cu") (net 30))
 (segment (start 146.795 50.205991) (end 146.795 49.274009) (width 0.25) (layer "F.Cu") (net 31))
 (segment (start 126 79.54) (end 124.825 78.365) (width 0.25) (layer "F.Cu") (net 31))
 (segment (start 140.606117 51.543883) (end 145.457108 51.543883) (width 0.25) (layer "F.Cu") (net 31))
 (segment (start 145.457108 51.543883) (end 146.795 50.205991) (width 0.25) (layer "F.Cu") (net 31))
 (segment (start 149.335 48.615) (end 150.46 49.74) (width 0.25) (layer "F.Cu") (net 31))
 (segment (start 124.825 78.365) (end 124.825 67.325) (width 0.25) (layer "F.Cu") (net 31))
 (segment (start 147.454009 48.615) (end 149.335 48.615) (width 0.25) (layer "F.Cu") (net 31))
 (segment (start 146.795 49.274009) (end 147.454009 48.615) (width 0.25) (layer "F.Cu") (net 31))
 (segment (start 124.825 67.325) (end 140.606117 51.543883) (width 0.25) (layer "F.Cu") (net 31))
 (segment (start 186 77.42) (end 177.38 86.04) (width 0.25) (layer "F.Cu") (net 5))
 (segment (start 177.46 97.92) (end 177.38 98) (width 0.25) (layer "F.Cu") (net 5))
 (segment (start 177.38 86.04) (end 177.38 98) (width 0.25) (layer "F.Cu") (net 5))
 (segment (start 153.595 94.175) (end 162.175 94.175) (width 0.25) (layer "B.Cu") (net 33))
 (segment (start 169.8 95.5) (end 172.3 98) (width 0.25) (layer "B.Cu") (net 33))
 (segment (start 139 79.58) (end 153.595 94.175) (width 0.25) (layer "B.Cu") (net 33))
 (segment (start 163.5 95.5) (end 169.8 95.5) (width 0.25) (layer "B.Cu") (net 33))
 (segment (start 162.175 94.175) (end 163.5 95.5) (width 0.25) (layer "B.Cu") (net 33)))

